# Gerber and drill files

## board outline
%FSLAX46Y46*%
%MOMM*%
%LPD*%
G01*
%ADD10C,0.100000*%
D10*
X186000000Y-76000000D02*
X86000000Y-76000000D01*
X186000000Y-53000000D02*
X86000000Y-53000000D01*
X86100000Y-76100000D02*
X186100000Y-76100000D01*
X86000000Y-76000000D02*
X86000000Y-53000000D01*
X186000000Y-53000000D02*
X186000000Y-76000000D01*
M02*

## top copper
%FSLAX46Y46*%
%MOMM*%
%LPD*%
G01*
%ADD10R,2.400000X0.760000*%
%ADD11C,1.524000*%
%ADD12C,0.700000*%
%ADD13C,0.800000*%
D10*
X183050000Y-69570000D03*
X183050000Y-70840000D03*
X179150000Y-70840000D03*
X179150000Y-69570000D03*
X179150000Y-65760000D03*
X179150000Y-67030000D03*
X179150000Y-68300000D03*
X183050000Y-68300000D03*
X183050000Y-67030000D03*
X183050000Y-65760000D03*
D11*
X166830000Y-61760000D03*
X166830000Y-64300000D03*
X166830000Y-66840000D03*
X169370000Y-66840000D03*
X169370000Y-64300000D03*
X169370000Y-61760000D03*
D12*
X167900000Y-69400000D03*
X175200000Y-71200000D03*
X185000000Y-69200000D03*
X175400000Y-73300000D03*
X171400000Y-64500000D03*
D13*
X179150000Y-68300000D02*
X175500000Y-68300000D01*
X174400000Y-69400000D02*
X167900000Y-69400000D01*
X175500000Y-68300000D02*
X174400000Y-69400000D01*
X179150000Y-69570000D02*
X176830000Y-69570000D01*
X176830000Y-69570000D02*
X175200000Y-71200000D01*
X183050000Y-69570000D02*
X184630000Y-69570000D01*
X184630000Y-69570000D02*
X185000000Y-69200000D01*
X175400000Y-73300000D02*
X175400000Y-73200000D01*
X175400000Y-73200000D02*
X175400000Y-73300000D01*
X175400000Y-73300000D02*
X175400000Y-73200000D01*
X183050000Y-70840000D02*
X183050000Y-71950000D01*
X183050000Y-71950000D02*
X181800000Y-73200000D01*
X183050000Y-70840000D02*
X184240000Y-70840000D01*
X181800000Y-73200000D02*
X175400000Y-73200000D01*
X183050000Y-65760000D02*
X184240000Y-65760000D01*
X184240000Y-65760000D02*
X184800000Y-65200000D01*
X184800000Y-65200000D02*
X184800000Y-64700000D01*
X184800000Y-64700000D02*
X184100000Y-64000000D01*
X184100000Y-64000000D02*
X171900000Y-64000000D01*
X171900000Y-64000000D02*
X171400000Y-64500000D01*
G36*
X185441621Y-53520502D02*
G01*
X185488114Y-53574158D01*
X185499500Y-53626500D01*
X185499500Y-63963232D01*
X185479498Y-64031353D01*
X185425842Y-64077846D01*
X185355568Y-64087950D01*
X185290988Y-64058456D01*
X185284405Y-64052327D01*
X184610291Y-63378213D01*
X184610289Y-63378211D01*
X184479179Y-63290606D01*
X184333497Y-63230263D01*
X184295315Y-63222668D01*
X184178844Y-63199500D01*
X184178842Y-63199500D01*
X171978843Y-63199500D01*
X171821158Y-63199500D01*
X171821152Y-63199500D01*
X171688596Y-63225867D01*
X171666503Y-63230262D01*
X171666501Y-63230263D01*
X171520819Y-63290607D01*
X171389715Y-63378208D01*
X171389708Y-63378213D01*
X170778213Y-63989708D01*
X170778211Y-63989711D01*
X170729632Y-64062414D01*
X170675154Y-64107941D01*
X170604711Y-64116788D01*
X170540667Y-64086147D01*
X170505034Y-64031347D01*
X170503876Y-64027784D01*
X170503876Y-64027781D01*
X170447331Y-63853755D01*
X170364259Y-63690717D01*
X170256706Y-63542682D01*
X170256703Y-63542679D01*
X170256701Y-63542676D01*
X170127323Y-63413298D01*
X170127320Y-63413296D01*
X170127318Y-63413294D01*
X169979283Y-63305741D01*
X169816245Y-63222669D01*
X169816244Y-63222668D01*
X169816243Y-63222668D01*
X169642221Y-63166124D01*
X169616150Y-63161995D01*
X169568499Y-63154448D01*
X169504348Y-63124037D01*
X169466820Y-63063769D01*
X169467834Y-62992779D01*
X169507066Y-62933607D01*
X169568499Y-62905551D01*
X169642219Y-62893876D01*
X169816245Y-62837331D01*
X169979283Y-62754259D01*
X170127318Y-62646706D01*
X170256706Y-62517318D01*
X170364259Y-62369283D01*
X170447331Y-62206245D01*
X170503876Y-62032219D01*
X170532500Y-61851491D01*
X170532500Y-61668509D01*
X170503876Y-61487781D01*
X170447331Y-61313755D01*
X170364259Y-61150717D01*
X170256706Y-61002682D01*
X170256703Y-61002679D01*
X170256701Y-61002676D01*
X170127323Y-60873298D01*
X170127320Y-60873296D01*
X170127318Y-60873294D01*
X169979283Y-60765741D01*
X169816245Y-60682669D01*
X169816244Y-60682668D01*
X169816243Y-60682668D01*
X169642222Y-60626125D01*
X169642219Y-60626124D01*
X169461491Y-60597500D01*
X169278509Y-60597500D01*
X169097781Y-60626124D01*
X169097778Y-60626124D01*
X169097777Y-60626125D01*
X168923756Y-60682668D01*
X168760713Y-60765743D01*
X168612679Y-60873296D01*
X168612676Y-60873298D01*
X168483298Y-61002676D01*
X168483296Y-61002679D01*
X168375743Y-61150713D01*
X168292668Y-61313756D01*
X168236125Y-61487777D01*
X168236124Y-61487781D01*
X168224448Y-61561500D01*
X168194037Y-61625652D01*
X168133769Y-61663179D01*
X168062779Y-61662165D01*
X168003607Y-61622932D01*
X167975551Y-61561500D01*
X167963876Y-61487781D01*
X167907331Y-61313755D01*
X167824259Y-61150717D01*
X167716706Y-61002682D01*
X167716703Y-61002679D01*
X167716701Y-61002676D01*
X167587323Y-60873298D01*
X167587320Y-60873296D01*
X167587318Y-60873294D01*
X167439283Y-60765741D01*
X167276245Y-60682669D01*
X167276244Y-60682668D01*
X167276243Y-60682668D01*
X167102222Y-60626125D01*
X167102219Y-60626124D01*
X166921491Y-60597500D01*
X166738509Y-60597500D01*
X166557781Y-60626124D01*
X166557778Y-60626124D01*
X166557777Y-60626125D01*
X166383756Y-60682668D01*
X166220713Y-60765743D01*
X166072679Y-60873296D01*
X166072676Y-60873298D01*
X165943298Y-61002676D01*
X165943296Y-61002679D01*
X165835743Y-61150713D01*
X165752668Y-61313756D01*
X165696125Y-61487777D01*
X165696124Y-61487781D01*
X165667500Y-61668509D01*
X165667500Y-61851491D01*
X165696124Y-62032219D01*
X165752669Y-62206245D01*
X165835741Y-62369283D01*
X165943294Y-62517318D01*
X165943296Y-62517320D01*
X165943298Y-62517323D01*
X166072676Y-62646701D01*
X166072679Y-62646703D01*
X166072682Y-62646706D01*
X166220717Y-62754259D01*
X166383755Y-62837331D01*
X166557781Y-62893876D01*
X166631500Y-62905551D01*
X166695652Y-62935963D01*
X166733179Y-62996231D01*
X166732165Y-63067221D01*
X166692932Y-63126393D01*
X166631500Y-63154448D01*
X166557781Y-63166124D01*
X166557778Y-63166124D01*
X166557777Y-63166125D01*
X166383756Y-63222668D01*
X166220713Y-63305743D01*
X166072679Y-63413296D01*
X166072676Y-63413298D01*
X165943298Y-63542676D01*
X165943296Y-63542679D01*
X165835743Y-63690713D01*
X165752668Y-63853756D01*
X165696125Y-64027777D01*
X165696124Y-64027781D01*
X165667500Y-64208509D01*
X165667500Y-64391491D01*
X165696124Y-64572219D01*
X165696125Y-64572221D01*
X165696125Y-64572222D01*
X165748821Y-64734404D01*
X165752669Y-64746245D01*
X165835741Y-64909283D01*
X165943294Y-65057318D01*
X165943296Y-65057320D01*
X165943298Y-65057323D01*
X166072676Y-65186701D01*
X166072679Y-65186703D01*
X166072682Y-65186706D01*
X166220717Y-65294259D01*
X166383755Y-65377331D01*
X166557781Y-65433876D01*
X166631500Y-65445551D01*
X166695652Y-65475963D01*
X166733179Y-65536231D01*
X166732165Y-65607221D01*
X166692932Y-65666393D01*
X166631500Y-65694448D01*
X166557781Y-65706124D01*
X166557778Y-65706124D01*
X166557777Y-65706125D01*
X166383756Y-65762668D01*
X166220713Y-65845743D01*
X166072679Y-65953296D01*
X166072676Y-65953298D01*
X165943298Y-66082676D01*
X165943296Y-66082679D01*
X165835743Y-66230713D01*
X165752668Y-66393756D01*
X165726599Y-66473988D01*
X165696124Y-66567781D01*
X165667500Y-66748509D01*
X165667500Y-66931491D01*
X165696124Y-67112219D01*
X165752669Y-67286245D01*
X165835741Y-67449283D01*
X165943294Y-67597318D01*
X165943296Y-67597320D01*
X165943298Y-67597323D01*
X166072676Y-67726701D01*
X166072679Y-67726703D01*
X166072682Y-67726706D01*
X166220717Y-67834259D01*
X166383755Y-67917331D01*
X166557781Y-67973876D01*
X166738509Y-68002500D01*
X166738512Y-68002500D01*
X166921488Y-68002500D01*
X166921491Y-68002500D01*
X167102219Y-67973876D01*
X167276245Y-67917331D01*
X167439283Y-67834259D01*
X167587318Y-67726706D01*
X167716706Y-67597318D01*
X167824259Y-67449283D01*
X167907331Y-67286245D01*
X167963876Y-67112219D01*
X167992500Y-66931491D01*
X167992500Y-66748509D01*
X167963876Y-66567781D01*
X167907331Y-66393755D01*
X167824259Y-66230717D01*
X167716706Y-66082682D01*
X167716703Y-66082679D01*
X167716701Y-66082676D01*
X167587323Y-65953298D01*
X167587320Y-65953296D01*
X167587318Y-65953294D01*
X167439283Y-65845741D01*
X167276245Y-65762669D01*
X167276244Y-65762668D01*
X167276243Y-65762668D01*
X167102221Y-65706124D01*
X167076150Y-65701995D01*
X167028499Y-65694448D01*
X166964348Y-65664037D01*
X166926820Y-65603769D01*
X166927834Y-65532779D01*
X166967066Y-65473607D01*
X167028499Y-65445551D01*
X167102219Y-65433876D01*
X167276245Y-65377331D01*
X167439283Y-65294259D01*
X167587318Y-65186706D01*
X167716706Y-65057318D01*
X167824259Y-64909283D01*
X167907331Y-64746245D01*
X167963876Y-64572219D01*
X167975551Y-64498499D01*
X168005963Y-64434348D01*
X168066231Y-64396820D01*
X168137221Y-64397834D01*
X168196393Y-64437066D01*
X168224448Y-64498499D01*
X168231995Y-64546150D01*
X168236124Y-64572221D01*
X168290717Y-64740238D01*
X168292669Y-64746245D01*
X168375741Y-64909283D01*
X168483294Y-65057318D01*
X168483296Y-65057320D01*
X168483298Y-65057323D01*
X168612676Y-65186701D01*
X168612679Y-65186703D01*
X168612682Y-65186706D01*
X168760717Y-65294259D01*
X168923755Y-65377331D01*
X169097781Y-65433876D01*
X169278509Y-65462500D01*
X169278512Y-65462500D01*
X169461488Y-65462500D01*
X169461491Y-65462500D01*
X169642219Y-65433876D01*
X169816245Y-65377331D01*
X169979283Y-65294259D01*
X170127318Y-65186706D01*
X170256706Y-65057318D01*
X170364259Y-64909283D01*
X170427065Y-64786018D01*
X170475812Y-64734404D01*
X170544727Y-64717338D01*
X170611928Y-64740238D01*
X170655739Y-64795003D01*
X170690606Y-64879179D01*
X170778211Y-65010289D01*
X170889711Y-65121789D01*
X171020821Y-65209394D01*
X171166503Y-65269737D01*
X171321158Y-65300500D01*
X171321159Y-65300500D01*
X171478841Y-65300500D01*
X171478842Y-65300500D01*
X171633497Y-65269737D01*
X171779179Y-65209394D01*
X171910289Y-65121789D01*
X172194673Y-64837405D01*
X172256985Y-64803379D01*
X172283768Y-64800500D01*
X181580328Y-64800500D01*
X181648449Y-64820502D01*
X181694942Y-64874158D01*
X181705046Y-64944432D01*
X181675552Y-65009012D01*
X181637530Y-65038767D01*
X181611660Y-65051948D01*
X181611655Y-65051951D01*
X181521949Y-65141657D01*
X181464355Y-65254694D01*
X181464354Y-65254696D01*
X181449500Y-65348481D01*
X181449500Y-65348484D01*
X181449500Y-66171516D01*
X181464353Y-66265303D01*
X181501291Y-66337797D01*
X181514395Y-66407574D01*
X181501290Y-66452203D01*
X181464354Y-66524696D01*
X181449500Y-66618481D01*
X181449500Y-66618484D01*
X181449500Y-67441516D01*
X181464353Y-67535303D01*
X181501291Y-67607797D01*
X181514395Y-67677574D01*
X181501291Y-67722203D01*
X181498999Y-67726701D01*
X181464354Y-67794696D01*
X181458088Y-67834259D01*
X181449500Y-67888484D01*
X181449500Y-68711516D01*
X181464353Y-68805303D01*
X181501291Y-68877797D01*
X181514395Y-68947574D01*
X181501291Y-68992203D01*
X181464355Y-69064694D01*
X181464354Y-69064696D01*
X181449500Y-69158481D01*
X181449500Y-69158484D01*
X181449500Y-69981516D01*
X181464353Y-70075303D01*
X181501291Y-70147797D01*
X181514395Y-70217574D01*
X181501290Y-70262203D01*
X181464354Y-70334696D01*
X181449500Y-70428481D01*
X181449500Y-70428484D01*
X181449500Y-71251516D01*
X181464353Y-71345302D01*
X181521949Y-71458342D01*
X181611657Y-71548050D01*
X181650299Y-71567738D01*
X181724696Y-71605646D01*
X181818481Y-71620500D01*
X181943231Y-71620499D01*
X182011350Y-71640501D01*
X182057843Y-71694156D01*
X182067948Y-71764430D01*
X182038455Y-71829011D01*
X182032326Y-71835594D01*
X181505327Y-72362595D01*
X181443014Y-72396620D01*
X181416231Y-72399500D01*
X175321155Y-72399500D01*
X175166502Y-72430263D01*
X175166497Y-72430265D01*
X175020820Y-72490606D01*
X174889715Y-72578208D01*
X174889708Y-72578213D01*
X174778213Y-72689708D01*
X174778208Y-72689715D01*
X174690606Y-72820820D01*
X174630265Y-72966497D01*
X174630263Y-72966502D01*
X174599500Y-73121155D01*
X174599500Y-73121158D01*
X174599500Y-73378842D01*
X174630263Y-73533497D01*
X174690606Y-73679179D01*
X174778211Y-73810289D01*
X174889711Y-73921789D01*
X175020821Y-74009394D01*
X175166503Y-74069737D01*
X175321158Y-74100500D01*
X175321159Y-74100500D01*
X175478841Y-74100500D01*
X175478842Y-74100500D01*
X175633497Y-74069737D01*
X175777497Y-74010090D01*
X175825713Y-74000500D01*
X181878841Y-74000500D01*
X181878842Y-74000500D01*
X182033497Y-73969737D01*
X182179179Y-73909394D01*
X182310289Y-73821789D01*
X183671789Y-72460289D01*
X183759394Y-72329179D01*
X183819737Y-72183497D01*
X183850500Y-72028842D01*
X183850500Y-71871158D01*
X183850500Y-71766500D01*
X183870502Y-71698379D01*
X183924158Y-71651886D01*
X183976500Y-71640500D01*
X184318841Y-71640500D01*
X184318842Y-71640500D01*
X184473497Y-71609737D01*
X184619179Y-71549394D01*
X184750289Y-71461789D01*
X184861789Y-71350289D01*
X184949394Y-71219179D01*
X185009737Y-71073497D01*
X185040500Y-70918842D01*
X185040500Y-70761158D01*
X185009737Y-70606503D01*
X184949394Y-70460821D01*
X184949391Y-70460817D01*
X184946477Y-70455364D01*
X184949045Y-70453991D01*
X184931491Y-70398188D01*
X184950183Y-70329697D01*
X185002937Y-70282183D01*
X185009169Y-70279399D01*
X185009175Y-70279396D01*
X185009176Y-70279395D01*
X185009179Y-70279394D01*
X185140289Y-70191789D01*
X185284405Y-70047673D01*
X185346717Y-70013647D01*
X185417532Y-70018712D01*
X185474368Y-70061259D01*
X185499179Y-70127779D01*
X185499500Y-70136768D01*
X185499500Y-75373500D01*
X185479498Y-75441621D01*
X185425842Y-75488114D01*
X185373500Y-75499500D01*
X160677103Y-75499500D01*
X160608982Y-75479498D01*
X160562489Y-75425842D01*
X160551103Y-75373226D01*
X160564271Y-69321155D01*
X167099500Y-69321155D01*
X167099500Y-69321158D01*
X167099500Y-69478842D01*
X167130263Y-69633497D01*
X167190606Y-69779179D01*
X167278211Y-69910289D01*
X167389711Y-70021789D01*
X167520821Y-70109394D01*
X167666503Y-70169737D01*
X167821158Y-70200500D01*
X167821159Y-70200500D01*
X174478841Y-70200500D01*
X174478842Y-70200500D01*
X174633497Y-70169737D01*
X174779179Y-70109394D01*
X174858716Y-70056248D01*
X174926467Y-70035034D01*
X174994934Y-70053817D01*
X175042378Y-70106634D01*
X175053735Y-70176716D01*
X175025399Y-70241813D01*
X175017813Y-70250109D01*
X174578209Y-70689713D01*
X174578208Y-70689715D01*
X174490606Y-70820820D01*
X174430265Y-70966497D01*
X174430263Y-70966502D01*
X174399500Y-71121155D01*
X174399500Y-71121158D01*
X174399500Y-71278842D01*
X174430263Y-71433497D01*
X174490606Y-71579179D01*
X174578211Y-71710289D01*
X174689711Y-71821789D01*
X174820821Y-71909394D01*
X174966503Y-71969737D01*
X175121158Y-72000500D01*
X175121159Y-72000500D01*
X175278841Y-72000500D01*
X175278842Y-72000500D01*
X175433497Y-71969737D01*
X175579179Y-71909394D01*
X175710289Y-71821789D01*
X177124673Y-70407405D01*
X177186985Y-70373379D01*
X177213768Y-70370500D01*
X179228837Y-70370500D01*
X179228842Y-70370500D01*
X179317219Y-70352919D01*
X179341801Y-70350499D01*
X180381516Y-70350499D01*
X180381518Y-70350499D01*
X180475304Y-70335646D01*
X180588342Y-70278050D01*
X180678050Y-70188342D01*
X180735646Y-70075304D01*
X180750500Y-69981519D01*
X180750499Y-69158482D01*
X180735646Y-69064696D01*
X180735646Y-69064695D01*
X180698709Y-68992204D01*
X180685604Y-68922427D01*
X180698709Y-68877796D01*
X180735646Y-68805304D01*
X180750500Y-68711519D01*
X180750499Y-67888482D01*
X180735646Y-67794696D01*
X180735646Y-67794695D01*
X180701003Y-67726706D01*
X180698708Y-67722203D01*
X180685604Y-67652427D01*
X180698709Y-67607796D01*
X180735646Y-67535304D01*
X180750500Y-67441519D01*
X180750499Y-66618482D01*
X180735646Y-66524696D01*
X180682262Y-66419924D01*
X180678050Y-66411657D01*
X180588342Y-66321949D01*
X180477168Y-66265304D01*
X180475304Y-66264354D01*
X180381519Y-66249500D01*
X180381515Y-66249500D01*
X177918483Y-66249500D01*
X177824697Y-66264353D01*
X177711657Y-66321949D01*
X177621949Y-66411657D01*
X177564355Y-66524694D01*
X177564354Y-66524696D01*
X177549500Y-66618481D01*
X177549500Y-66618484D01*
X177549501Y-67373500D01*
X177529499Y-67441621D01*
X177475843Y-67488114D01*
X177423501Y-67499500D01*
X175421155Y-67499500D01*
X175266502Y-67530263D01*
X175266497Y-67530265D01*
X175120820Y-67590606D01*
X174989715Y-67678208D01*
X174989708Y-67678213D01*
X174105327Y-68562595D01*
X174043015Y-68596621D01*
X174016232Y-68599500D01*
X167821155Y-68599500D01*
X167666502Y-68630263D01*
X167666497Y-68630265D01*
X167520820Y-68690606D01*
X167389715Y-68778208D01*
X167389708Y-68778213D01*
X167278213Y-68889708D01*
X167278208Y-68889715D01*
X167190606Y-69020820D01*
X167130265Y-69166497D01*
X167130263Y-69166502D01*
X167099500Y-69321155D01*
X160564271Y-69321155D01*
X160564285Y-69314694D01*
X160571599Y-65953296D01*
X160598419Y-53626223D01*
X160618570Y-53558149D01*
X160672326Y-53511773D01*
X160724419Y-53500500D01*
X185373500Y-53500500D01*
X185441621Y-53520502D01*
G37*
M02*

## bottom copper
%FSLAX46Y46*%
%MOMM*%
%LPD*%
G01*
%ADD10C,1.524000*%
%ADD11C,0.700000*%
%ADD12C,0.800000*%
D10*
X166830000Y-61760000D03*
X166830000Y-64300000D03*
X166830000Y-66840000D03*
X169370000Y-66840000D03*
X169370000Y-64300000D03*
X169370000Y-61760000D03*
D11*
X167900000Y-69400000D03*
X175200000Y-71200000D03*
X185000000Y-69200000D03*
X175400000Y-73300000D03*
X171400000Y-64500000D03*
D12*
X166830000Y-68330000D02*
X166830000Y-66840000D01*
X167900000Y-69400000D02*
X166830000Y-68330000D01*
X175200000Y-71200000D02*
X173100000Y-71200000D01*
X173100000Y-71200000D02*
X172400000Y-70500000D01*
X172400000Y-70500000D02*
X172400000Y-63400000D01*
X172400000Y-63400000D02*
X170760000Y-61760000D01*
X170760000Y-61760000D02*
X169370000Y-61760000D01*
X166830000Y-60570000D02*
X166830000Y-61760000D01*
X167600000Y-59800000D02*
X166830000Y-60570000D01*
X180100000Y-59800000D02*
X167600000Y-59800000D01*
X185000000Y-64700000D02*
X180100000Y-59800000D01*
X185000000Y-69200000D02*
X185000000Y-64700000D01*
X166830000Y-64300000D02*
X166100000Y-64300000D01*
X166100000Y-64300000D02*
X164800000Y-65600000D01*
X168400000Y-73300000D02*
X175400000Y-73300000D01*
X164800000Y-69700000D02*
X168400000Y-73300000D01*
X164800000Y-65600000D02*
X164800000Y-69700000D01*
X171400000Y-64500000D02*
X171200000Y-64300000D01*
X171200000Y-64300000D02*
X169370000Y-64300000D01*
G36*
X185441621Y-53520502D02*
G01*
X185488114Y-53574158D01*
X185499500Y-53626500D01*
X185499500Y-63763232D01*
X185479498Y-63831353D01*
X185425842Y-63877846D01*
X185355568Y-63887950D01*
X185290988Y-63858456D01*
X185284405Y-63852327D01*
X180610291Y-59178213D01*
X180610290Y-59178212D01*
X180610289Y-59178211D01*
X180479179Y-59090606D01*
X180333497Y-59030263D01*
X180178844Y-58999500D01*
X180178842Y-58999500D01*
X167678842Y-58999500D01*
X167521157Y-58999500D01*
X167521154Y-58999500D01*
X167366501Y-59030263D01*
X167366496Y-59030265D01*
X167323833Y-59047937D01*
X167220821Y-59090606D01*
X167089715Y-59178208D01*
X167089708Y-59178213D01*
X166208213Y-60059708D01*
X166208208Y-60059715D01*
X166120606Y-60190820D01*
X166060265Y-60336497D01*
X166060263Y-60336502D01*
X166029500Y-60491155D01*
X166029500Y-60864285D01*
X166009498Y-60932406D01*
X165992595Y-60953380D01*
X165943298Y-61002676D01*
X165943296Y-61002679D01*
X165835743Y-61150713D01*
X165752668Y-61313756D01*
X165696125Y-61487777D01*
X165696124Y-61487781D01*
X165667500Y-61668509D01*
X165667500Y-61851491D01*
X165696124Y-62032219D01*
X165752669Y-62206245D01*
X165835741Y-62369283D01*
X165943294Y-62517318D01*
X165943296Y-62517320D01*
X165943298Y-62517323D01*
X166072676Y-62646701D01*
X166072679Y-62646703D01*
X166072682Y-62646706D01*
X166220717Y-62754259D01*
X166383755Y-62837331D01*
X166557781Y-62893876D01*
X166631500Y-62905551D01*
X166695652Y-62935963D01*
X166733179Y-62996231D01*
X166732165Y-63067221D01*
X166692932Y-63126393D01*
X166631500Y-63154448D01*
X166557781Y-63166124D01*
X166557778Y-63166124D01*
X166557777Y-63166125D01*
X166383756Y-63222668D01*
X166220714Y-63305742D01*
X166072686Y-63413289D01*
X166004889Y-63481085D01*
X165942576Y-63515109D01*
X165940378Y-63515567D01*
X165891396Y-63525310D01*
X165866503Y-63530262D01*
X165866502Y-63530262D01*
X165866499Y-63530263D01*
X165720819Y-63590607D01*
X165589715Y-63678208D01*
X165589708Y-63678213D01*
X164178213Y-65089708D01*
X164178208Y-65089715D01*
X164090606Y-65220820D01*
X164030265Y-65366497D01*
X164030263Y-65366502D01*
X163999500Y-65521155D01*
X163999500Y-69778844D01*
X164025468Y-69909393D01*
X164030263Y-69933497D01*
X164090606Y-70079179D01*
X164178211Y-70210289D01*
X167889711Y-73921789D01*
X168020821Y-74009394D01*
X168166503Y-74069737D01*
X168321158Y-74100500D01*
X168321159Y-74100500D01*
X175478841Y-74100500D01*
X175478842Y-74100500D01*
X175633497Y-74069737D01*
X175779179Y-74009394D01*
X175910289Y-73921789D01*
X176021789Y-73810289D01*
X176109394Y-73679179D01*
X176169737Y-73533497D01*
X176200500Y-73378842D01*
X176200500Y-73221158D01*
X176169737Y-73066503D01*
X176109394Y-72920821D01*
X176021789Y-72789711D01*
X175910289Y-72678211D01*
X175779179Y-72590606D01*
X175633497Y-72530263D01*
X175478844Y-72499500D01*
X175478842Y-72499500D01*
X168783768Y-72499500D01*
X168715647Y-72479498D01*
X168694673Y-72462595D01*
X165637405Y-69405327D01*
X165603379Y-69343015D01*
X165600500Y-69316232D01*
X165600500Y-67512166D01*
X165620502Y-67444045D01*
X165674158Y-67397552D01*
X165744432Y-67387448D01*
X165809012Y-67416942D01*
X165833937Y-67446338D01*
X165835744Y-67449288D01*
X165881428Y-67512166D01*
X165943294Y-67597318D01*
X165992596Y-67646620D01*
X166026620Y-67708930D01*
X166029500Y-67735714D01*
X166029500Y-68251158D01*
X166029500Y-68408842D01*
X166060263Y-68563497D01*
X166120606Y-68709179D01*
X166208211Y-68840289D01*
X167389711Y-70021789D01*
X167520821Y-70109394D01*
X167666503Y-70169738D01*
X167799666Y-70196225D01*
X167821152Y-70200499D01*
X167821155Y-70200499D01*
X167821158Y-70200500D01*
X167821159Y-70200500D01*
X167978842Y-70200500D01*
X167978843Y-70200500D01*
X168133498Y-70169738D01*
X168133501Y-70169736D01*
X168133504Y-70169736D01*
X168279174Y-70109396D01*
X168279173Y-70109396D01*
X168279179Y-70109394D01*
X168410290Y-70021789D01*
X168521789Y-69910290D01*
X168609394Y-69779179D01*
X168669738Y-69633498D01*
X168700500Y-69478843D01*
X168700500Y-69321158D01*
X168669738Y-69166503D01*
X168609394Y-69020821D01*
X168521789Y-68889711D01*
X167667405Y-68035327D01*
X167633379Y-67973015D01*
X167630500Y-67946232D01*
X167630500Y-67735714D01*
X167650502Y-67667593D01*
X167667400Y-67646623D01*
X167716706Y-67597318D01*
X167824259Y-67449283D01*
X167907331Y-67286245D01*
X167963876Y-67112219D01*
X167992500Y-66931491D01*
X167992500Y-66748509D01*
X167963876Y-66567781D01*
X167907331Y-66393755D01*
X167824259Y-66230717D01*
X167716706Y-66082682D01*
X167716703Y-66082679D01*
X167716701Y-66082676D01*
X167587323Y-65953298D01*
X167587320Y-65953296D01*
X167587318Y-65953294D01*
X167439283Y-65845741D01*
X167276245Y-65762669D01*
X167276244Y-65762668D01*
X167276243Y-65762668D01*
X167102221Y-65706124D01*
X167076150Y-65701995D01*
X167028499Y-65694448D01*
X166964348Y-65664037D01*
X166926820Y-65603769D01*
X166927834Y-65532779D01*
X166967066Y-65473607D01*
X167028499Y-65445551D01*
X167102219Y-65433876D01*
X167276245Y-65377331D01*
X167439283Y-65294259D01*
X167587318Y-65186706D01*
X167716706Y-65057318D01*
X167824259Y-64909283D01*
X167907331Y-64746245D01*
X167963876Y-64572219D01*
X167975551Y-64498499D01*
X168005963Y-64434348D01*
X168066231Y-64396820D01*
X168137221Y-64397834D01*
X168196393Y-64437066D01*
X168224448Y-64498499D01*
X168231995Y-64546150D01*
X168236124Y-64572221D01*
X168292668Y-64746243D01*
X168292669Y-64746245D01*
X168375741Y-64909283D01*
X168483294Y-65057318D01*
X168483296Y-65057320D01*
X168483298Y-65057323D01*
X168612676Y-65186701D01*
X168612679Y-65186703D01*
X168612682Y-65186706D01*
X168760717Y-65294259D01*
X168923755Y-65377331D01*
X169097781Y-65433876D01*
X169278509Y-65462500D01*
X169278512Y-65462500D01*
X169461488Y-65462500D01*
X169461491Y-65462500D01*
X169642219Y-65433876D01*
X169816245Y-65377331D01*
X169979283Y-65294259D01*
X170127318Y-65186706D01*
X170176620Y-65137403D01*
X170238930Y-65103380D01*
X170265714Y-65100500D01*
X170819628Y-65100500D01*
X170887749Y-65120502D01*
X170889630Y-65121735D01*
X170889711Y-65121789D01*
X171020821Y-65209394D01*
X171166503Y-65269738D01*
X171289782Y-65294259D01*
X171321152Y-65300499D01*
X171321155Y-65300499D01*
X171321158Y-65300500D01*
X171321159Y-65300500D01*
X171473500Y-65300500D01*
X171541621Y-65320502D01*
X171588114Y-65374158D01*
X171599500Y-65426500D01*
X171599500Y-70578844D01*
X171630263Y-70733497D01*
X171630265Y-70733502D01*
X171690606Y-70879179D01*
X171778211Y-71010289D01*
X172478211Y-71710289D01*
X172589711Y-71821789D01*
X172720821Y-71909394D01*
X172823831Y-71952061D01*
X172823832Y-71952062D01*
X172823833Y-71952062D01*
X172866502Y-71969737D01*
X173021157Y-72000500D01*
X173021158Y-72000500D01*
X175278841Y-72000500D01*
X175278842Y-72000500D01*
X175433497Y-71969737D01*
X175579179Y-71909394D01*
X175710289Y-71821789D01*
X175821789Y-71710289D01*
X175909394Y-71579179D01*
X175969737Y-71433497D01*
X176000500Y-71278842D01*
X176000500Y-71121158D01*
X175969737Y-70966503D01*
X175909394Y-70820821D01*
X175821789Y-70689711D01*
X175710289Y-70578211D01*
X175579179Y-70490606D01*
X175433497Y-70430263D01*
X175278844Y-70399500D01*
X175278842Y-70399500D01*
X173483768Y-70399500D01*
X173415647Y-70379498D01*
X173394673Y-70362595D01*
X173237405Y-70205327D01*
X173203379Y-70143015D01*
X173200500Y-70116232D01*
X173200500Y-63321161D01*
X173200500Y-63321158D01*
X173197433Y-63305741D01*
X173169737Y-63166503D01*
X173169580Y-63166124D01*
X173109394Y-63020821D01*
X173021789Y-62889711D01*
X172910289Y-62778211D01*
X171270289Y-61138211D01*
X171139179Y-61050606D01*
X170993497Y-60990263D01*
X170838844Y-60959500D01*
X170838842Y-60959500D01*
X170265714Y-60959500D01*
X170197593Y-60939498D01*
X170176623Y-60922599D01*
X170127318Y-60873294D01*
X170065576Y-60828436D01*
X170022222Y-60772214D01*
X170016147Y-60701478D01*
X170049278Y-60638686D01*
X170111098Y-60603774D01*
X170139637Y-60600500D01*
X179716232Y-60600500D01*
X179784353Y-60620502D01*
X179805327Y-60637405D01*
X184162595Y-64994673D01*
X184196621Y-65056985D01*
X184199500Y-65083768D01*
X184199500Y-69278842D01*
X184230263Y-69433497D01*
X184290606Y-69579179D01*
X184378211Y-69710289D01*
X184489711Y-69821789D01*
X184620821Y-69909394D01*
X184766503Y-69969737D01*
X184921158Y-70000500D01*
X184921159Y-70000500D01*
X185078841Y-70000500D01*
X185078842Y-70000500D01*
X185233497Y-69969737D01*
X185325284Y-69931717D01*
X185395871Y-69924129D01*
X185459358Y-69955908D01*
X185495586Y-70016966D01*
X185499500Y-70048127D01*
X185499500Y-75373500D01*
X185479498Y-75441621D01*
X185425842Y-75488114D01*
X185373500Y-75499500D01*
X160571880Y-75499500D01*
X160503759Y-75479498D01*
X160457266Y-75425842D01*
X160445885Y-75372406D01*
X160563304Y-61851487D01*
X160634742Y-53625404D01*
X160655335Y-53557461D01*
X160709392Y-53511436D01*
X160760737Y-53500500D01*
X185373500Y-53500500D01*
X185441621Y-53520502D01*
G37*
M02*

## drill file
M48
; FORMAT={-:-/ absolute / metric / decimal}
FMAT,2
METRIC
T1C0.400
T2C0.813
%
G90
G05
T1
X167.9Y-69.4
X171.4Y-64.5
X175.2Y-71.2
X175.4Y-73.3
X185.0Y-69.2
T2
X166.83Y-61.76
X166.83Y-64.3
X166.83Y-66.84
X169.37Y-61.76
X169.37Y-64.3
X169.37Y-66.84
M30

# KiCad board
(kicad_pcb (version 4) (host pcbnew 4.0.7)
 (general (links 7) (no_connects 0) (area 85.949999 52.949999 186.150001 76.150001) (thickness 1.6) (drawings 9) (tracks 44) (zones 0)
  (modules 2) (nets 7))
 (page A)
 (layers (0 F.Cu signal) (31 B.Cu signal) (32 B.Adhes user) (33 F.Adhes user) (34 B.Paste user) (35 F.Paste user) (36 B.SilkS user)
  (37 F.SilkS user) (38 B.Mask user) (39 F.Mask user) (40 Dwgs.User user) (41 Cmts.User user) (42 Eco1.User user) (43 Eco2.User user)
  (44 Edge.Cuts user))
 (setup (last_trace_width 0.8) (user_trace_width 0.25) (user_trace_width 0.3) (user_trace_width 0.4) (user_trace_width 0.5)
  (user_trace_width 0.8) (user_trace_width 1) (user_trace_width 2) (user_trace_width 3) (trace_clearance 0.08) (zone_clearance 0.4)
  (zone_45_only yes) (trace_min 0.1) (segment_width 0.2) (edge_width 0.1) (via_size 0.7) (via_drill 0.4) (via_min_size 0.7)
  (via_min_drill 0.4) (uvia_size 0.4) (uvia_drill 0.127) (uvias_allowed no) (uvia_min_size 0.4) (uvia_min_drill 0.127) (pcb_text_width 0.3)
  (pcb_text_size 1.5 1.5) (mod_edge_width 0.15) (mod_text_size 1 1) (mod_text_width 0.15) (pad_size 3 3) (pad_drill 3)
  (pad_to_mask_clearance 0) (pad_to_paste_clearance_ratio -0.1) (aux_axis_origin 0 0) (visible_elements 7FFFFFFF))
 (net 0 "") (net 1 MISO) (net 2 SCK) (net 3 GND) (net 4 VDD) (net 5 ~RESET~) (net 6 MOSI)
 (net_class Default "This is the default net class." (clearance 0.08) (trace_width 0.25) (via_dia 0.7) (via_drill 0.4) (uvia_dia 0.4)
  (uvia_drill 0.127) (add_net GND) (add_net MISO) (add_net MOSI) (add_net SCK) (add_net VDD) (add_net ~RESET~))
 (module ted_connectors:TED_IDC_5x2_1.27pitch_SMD (layer F.Cu) (at 181.1 68.3 270)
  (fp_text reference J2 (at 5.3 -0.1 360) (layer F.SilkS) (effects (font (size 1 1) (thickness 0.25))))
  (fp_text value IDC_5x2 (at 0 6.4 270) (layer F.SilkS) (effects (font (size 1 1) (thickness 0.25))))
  (pad 8 smd rect (at 1.27 -1.95 270) (size 0.76 2.4) (layers F.Cu F.Paste F.Mask) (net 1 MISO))
  (pad 10 smd rect (at 2.54 -1.95 270) (size 0.76 2.4) (layers F.Cu F.Paste F.Mask) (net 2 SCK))
  (pad 9 smd rect (at 2.54 1.95 270) (size 0.76 2.4) (layers F.Cu F.Paste F.Mask) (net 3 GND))
  (pad 7 smd rect (at 1.27 1.95 270) (size 0.76 2.4) (layers F.Cu F.Paste F.Mask) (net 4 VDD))
  (pad 1 smd rect (at -2.54 1.95 270) (size 0.76 2.4) (layers F.Cu F.Paste F.Mask) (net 3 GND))
  (pad 3 smd rect (at -1.27 1.95 270) (size 0.76 2.4) (layers F.Cu F.Paste F.Mask))
  (pad 5 smd rect (at 0 1.95 270) (size 0.76 2.4) (layers F.Cu F.Paste F.Mask) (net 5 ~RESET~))
  (pad 6 smd rect (at 0 -1.95 270) (size 0.76 2.4) (layers F.Cu F.Paste F.Mask))
  (pad 4 smd rect (at -1.27 -1.95 270) (size 0.76 2.4) (layers F.Cu F.Paste F.Mask))
  (pad 2 smd rect (at -2.54 -1.95 270) (size 0.76 2.4) (layers F.Cu F.Paste F.Mask) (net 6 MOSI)))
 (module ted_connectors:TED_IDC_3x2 (layer F.Cu) (at 168.1 64.3 270)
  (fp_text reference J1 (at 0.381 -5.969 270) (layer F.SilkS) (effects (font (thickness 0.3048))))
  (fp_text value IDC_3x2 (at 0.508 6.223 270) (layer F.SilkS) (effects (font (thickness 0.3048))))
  (pad 1 thru_hole circle (at -2.54 1.27 270) (size 1.524 1.524) (drill 0.8128) (layers *.Cu *.Mask F.SilkS) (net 1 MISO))
  (pad 3 thru_hole circle (at 0 1.27 270) (size 1.524 1.524) (drill 0.8128) (layers *.Cu *.Mask F.SilkS) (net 2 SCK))
  (pad 5 thru_hole circle (at 2.54 1.27 270) (size 1.524 1.524) (drill 0.8128) (layers *.Cu *.Mask F.SilkS) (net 5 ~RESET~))
  (pad 6 thru_hole circle (at 2.54 -1.27 270) (size 1.524 1.524) (drill 0.8128) (layers *.Cu *.Mask F.SilkS) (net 3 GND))
  (pad 4 thru_hole circle (at 0 -1.27 270) (size 1.524 1.524) (drill 0.8128) (layers *.Cu *.Mask F.SilkS) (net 6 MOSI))
  (pad 2 thru_hole circle (at -2.54 -1.27 270) (size 1.524 1.524) (drill 0.8128) (layers *.Cu *.Mask F.SilkS) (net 4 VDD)))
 (gr_line (start 186 76) (end 86 76) (angle 90) (layer Edge.Cuts) (width 0.1))
 (gr_line (start 186 53) (end 86 53) (angle 90) (layer Edge.Cuts) (width 0.1))
 (gr_line (start 86.1 76.1) (end 186.1 76.1) (angle 90) (layer Edge.Cuts) (width 0.1))
 (gr_line (start 86 76) (end 86 53) (angle 90) (layer Edge.Cuts) (width 0.1))
 (gr_line (start 186 53) (end 186 76) (angle 90) (layer Edge.Cuts) (width 0.1))
 (segment (start 179.15 68.3) (end 175.5 68.3) (width 0.8) (layer F.Cu) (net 5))
 (segment (start 166.83 68.33) (end 166.83 66.84) (width 0.8) (layer B.Cu) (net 5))
 (segment (start 167.9 69.4) (end 166.83 68.33) (width 0.8) (layer B.Cu) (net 5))
 (via (at 167.9 69.4) (size 0.7) (drill 0.4) (layers F.Cu B.Cu) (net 5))
 (segment (start 174.4 69.4) (end 167.9 69.4) (width 0.8) (layer F.Cu) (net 5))
 (segment (start 175.5 68.3) (end 174.4 69.4) (width 0.8) (layer F.Cu) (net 5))
 (segment (start 179.15 69.57) (end 176.83 69.57) (width 0.8) (layer F.Cu) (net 4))
 (segment (start 176.83 69.57) (end 175.2 71.2) (width 0.8) (layer F.Cu) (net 4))
 (via (at 175.2 71.2) (size 0.7) (drill 0.4) (layers F.Cu B.Cu) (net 4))
 (segment (start 175.2 71.2) (end 173.1 71.2) (width 0.8) (layer B.Cu) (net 4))
 (segment (start 173.1 71.2) (end 172.4 70.5) (width 0.8) (layer B.Cu) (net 4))
 (segment (start 172.4 70.5) (end 172.4 63.4) (width 0.8) (layer B.Cu) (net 4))
 (segment (start 172.4 63.4) (end 170.76 61.76) (width 0.8) (layer B.Cu) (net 4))
 (segment (start 170.76 61.76) (end 169.37 61.76) (width 0.8) (layer B.Cu) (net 4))
 (segment (start 183.05 69.57) (end 184.63 69.57) (width 0.8) (layer F.Cu) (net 1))
 (segment (start 166.83 60.57) (end 166.83 61.76) (width 0.8) (layer B.Cu) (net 1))
 (segment (start 167.6 59.8) (end 166.83 60.57) (width 0.8) (layer B.Cu) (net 1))
 (segment (start 180.1 59.8) (end 167.6 59.8) (width 0.8) (layer B.Cu) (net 1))
 (segment (start 185 64.7) (end 180.1 59.8) (width 0.8) (layer B.Cu) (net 1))
 (segment (start 185 69.2) (end 185 64.7) (width 0.8) (layer B.Cu) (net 1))
 (via (at 185 69.2) (size 0.7) (drill 0.4) (layers F.Cu B.Cu) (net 1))
 (segment (start 184.63 69.57) (end 185 69.2) (width 0.8) (layer F.Cu) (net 1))
 (segment (start 166.83 64.3) (end 166.1 64.3) (width 0.8) (layer B.Cu) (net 2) (status C00000))
 (segment (start 166.1 64.3) (end 164.8 65.6) (width 0.8) (layer B.Cu) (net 2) (status 400000))
 (via (at 175.4 73.3) (size 0.7) (drill 0.4) (layers F.Cu B.Cu) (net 2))
 (segment (start 168.4 73.3) (end 175.4 73.3) (width 0.8) (layer B.Cu) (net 2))
 (segment (start 164.8 69.7) (end 168.4 73.3) (width 0.8) (layer B.Cu) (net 2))
 (segment (start 164.8 65.6) (end 164.8 69.7) (width 0.8) (layer B.Cu) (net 2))
 (segment (start 175.4 73.3) (end 175.4 73.2) (width 0.8) (layer F.Cu) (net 2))
 (segment (start 175.4 73.2) (end 175.4 73.3) (width 0.8) (layer F.Cu) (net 2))
 (segment (start 175.4 73.3) (end 175.4 73.2) (width 0.8) (layer F.Cu) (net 2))
 (segment (start 183.05 70.84) (end 183.05 71.95) (width 0.8) (layer F.Cu) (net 2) (status 400000))
 (segment (start 183.05 71.95) (end 181.8 73.2) (width 0.8) (layer F.Cu) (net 2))
 (segment (start 183.05 70.84) (end 184.24 70.84) (width 0.8) (layer F.Cu) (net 2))
 (segment (start 181.8 73.2) (end 175.4 73.2) (width 0.8) (layer F.Cu) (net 2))
 (segment (start 183.05 65.76) (end 184.24 65.76) (width 0.8) (layer F.Cu) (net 6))
 (segment (start 184.24 65.76) (end 184.8 65.2) (width 0.8) (layer F.Cu) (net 6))
 (segment (start 184.8 65.2) (end 184.8 64.7) (width 0.8) (layer F.Cu) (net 6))
 (segment (start 184.8 64.7) (end 184.1 64) (width 0.8) (layer F.Cu) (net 6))
 (segment (start 184.1 64) (end 171.9 64) (width 0.8) (layer F.Cu) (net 6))
 (segment (start 171.9 64) (end 171.4 64.5) (width 0.8) (layer F.Cu) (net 6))
 (via (at 171.4 64.5) (size 0.7) (drill 0.4) (layers F.Cu B.Cu) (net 6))
 (segment (start 171.4 64.5) (end 171.2 64.3) (width 0.8) (layer B.Cu) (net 6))
 (segment (start 171.2 64.3) (end 169.37 64.3) (width 0.8) (layer B.Cu) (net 6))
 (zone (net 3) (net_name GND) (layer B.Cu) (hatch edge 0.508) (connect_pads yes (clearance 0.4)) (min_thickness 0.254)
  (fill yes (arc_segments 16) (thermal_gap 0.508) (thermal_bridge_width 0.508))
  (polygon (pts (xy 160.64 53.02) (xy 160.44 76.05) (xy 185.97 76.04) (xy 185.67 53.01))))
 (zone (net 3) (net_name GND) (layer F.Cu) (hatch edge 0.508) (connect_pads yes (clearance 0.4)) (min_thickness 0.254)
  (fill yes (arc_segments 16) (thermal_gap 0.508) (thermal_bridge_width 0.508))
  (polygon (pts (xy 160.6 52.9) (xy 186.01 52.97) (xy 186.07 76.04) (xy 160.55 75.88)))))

